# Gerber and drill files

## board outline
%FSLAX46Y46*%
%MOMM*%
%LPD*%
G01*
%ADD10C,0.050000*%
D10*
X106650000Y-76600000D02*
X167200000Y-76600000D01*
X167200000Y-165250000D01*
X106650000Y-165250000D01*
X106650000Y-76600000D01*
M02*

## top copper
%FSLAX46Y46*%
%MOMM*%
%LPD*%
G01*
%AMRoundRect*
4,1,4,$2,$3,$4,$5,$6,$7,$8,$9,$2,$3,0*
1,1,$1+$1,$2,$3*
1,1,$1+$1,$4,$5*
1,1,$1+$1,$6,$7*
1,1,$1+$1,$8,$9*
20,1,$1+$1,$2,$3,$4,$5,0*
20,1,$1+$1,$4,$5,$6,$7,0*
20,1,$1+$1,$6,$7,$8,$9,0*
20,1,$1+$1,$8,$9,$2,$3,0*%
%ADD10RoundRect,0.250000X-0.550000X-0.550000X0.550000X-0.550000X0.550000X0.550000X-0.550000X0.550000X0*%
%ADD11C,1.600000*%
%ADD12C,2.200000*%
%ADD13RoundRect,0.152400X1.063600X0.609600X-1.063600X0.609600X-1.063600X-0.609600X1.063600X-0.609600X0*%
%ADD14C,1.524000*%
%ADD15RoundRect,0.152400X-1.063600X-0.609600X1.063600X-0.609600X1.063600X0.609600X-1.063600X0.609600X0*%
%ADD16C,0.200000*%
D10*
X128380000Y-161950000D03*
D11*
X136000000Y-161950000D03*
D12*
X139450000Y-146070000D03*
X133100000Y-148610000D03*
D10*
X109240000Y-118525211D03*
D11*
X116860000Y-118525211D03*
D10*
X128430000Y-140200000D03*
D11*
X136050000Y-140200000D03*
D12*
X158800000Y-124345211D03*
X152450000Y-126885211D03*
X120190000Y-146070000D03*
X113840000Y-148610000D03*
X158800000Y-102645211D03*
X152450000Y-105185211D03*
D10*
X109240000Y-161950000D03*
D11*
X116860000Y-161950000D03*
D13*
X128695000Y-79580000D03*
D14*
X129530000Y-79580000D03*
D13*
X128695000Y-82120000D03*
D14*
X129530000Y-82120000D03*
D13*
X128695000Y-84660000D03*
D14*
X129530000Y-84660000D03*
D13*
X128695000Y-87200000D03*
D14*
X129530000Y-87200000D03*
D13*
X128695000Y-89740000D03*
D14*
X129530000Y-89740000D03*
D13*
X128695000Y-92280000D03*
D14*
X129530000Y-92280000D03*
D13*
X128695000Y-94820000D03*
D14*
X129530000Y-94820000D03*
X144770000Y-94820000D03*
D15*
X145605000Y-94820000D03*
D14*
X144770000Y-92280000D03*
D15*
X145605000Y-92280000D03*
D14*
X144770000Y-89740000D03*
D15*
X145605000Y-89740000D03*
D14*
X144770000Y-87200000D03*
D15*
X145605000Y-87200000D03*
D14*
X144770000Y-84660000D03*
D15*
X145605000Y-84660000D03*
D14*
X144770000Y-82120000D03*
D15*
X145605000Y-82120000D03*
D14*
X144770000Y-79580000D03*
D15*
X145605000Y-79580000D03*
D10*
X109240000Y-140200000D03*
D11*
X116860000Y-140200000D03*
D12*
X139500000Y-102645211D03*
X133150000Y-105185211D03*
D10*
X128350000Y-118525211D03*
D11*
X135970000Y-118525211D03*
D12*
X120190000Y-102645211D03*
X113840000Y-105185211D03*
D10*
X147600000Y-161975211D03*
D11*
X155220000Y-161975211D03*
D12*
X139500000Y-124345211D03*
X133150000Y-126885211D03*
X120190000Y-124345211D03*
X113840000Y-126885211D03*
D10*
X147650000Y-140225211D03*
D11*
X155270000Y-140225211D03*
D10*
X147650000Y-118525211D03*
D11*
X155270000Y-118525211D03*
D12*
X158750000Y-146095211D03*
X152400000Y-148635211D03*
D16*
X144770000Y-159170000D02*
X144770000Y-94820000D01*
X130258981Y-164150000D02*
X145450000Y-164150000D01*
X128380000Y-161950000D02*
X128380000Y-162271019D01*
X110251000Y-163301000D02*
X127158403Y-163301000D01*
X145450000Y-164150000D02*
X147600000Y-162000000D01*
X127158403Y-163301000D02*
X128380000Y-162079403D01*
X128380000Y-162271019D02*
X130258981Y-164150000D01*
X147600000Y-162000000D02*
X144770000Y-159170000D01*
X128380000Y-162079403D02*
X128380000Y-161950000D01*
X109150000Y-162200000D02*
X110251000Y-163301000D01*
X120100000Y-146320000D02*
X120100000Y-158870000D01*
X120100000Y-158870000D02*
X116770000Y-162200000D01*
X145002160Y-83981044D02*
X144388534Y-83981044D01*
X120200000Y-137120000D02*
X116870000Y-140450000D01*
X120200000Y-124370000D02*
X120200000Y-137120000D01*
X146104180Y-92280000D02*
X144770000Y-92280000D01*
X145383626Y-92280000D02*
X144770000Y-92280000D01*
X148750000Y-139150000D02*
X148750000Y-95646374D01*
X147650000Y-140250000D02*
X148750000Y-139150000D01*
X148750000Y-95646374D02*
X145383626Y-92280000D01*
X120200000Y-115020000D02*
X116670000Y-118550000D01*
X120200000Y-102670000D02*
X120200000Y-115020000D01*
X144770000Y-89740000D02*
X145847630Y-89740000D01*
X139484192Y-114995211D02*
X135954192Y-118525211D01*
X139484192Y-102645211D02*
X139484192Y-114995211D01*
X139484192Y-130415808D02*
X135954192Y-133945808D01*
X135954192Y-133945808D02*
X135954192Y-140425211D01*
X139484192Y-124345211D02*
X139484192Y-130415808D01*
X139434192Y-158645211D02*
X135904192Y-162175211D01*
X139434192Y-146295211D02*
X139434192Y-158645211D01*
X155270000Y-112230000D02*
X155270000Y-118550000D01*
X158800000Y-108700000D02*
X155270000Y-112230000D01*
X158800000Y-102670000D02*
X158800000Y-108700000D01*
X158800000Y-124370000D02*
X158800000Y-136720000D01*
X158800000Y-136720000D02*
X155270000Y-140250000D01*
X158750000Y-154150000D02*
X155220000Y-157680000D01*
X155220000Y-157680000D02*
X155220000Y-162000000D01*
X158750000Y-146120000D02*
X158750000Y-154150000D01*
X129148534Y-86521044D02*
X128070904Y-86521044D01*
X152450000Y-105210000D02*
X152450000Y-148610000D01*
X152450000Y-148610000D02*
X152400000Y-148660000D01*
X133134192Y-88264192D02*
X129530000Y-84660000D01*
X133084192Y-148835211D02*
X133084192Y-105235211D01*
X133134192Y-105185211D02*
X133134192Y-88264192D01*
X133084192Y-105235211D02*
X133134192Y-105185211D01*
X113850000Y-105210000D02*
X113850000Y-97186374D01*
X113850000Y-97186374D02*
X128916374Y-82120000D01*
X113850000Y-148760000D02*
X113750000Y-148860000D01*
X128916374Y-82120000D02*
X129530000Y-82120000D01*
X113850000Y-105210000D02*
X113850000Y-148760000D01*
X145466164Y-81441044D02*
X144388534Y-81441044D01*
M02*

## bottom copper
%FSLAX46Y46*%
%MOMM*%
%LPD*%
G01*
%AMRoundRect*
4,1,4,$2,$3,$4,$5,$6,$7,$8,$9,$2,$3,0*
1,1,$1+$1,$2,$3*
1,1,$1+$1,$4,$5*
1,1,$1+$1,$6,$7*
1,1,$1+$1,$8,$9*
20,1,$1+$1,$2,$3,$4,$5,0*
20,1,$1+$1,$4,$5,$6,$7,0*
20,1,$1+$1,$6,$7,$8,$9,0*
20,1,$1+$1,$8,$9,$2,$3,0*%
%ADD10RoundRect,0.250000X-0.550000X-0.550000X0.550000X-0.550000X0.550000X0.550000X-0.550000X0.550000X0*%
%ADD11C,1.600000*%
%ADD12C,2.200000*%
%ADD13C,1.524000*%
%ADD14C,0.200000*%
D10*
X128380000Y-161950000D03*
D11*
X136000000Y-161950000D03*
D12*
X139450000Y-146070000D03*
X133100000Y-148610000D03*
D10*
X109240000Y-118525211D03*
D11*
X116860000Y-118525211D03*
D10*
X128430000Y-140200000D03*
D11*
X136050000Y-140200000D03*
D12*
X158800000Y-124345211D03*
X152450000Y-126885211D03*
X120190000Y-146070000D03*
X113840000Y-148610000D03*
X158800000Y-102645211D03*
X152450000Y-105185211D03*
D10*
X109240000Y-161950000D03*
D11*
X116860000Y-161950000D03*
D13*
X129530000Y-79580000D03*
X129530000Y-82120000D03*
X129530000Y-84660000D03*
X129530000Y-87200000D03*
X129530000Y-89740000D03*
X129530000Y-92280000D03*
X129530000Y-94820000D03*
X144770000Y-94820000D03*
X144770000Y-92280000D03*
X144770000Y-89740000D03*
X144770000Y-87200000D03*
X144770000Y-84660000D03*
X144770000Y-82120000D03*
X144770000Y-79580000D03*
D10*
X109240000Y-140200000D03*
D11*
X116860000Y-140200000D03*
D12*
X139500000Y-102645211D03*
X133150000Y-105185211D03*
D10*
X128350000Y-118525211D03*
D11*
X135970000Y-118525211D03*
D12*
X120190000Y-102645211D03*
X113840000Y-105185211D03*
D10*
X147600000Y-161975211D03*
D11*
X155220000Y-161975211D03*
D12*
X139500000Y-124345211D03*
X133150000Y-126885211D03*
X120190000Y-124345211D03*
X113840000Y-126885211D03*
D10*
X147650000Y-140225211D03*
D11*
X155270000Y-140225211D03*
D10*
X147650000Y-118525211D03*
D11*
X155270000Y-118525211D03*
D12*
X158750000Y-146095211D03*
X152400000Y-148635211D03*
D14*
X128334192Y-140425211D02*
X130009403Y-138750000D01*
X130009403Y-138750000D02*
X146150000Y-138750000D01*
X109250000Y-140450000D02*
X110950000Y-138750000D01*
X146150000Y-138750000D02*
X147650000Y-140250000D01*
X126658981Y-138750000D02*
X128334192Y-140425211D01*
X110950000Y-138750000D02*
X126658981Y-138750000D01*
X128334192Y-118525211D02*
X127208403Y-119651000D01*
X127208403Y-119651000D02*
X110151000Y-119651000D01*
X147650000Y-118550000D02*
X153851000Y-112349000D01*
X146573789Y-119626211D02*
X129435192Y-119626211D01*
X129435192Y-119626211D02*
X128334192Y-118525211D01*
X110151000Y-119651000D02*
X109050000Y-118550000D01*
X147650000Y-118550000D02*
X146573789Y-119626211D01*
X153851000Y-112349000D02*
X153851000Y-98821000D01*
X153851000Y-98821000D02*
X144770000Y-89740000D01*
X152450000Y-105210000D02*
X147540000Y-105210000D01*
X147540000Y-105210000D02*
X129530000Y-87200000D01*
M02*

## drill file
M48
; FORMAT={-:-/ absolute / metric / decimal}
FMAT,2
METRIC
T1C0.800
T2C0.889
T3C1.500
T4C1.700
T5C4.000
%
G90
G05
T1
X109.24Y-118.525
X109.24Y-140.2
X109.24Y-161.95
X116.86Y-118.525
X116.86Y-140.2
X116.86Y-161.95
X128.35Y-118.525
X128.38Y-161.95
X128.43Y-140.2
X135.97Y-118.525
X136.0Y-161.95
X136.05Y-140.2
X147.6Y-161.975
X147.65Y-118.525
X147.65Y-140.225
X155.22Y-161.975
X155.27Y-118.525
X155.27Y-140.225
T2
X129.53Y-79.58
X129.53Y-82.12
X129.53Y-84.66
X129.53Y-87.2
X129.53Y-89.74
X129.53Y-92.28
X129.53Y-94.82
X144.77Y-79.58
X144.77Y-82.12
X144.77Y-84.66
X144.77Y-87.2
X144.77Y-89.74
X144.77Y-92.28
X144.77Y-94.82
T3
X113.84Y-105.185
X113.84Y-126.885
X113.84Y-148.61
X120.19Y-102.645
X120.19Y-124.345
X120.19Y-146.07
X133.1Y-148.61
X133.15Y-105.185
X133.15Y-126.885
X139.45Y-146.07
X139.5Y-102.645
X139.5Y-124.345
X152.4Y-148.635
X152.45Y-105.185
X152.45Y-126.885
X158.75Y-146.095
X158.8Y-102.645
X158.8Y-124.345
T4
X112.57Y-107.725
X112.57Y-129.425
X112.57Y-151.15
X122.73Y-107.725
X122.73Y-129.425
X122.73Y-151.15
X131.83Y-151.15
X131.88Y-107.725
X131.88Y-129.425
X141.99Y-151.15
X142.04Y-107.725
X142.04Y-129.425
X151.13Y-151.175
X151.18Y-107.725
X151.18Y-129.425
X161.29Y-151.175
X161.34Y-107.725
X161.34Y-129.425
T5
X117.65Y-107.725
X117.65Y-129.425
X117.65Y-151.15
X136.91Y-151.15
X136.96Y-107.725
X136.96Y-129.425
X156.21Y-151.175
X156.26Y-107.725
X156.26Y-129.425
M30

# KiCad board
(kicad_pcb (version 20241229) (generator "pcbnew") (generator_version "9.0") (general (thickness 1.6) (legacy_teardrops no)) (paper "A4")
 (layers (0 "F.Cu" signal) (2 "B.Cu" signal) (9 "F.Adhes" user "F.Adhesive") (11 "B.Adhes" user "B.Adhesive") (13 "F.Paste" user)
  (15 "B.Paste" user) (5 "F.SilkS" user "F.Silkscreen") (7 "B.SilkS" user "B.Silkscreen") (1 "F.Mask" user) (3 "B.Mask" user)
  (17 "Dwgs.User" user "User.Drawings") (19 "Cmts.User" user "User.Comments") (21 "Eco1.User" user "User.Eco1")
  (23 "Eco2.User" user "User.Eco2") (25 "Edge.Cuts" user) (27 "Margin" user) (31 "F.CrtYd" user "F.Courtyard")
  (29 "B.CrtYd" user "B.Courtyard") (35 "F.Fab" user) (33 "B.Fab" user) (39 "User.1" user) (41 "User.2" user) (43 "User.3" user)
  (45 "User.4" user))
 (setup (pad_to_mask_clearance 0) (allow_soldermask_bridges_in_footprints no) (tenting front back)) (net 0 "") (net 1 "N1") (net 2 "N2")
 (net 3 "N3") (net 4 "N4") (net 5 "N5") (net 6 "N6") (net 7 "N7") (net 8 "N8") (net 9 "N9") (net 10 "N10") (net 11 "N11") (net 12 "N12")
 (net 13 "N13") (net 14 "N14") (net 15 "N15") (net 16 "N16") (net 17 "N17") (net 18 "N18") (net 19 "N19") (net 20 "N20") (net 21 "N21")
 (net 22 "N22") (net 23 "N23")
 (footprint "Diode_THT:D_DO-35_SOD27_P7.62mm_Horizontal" (layer "F.Cu") (at 128.38 161.95)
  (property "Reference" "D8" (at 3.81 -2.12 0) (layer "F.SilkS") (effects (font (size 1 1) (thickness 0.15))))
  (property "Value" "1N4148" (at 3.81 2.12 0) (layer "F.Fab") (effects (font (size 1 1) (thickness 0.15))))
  (pad "1" thru_hole roundrect (at 0 0) (size 1.6 1.6) (drill 0.8) (layers "*.Cu" "*.Mask") (remove_unused_layers no)
   (roundrect_rratio 0.15625) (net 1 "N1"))
  (pad "2" thru_hole circle (at 7.62 0) (size 1.6 1.6) (drill 0.8) (layers "*.Cu" "*.Mask") (remove_unused_layers no) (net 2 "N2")))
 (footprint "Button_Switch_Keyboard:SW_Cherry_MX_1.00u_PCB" (layer "F.Cu") (at 139.45 146.07)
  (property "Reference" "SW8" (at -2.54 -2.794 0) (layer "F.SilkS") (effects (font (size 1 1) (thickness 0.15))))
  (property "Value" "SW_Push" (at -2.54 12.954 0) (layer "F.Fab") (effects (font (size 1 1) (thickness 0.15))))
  (pad "" np_thru_hole circle (at -7.62 5.08) (size 1.7 1.7) (drill 1.7) (layers "*.Cu" "*.Mask"))
  (pad "" np_thru_hole circle (at -2.54 5.08) (size 4 4) (drill 4) (layers "*.Cu" "*.Mask"))
  (pad "" np_thru_hole circle (at 2.54 5.08) (size 1.7 1.7) (drill 1.7) (layers "*.Cu" "*.Mask"))
  (pad "1" thru_hole circle (at 0 0) (size 2.2 2.2) (drill 1.5) (layers "*.Cu" "*.Mask") (remove_unused_layers no) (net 2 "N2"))
  (pad "2" thru_hole circle (at -6.35 2.54) (size 2.2 2.2) (drill 1.5) (layers "*.Cu" "*.Mask") (remove_unused_layers no) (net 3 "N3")))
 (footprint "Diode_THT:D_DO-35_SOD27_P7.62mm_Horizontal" (layer "F.Cu") (at 109.24 118.525211)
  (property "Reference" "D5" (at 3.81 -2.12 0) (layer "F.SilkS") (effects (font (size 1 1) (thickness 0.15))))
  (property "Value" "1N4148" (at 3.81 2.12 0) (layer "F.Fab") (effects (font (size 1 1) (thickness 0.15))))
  (pad "1" thru_hole roundrect (at 0 0) (size 1.6 1.6) (drill 0.8) (layers "*.Cu" "*.Mask") (remove_unused_layers no)
   (roundrect_rratio 0.15625) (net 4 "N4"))
  (pad "2" thru_hole circle (at 7.62 0) (size 1.6 1.6) (drill 0.8) (layers "*.Cu" "*.Mask") (remove_unused_layers no) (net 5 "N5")))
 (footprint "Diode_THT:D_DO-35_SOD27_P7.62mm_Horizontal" (layer "F.Cu") (at 128.43 140.2)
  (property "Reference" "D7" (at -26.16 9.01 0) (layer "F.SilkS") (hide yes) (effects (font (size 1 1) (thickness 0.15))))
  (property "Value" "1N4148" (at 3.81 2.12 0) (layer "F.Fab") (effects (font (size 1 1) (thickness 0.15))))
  (pad "1" thru_hole roundrect (at 0 0) (size 1.6 1.6) (drill 0.8) (layers "*.Cu" "*.Mask") (remove_unused_layers no)
   (roundrect_rratio 0.15625) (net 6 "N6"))
  (pad "2" thru_hole circle (at 7.62 0) (size 1.6 1.6) (drill 0.8) (layers "*.Cu" "*.Mask") (remove_unused_layers no) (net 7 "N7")))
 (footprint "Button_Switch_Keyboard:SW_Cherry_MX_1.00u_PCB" (layer "F.Cu") (at 158.8 124.345211)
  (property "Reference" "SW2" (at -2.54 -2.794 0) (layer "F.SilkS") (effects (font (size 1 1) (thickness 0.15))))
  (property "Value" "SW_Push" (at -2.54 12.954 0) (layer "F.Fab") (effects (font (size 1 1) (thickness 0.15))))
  (pad "" np_thru_hole circle (at -7.62 5.08) (size 1.7 1.7) (drill 1.7) (layers "*.Cu" "*.Mask"))
  (pad "" np_thru_hole circle (at -2.54 5.08) (size 4 4) (drill 4) (layers "*.Cu" "*.Mask"))
  (pad "" np_thru_hole circle (at 2.54 5.08) (size 1.7 1.7) (drill 1.7) (layers "*.Cu" "*.Mask"))
  (pad "1" thru_hole circle (at 0 0) (size 2.2 2.2) (drill 1.5) (layers "*.Cu" "*.Mask") (remove_unused_layers no) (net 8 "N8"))
  (pad "2" thru_hole circle (at -6.35 2.54) (size 2.2 2.2) (drill 1.5) (layers "*.Cu" "*.Mask") (remove_unused_layers no) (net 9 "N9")))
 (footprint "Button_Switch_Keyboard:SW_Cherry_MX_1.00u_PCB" (layer "F.Cu") (at 120.19 146.07)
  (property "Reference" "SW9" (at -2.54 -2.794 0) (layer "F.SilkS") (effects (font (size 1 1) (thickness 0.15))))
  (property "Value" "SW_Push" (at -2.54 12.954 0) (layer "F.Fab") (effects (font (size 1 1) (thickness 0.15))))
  (pad "" np_thru_hole circle (at -7.62 5.08) (size 1.7 1.7) (drill 1.7) (layers "*.Cu" "*.Mask"))
  (pad "" np_thru_hole circle (at -2.54 5.08) (size 4 4) (drill 4) (layers "*.Cu" "*.Mask"))
  (pad "" np_thru_hole circle (at 2.54 5.08) (size 1.7 1.7) (drill 1.7) (layers "*.Cu" "*.Mask"))
  (pad "1" thru_hole circle (at 0 0) (size 2.2 2.2) (drill 1.5) (layers "*.Cu" "*.Mask") (remove_unused_layers no) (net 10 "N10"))
  (pad "2" thru_hole circle (at -6.35 2.54) (size 2.2 2.2) (drill 1.5) (layers "*.Cu" "*.Mask") (remove_unused_layers no) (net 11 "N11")))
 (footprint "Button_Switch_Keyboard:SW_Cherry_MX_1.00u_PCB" (layer "F.Cu") (at 158.8 102.645211)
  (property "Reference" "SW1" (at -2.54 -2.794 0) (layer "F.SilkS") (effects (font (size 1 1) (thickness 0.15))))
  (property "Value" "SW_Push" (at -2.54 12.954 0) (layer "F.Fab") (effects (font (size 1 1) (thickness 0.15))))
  (pad "" np_thru_hole circle (at -7.62 5.08) (size 1.7 1.7) (drill 1.7) (layers "*.Cu" "*.Mask"))
  (pad "" np_thru_hole circle (at -2.54 5.08) (size 4 4) (drill 4) (layers "*.Cu" "*.Mask"))
  (pad "" np_thru_hole circle (at 2.54 5.08) (size 1.7 1.7) (drill 1.7) (layers "*.Cu" "*.Mask"))
  (pad "1" thru_hole circle (at 0 0) (size 2.2 2.2) (drill 1.5) (layers "*.Cu" "*.Mask") (remove_unused_layers no) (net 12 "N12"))
  (pad "2" thru_hole circle (at -6.35 2.54) (size 2.2 2.2) (drill 1.5) (layers "*.Cu" "*.Mask") (remove_unused_layers no) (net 9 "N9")))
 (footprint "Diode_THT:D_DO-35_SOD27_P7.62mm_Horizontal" (layer "F.Cu") (at 109.24 161.95)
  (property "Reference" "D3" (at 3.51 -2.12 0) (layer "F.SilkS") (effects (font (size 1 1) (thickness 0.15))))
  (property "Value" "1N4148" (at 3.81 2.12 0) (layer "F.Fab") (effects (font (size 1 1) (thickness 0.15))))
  (pad "1" thru_hole roundrect (at 0 0) (size 1.6 1.6) (drill 0.8) (layers "*.Cu" "*.Mask") (remove_unused_layers no)
   (roundrect_rratio 0.15625) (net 1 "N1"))
  (pad "2" thru_hole circle (at 7.62 0) (size 1.6 1.6) (drill 0.8) (layers "*.Cu" "*.Mask") (remove_unused_layers no) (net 10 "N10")))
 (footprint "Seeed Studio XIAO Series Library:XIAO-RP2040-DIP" (layer "F.Cu") (at 137.15 87.2)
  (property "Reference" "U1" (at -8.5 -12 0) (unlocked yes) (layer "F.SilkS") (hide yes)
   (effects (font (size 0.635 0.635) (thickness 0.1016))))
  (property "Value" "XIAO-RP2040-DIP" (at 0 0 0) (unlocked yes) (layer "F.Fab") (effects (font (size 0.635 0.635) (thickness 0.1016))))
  (pad "1" smd roundrect (at -8.455 -7.62 180) (size 2.432 1.524) (layers "F.Cu" "F.Mask") (roundrect_rratio 0.1) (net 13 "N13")
   (thermal_bridge_angle 45))
  (pad "1" thru_hole circle (at -7.62 -7.62 180) (size 1.524 1.524) (drill 0.889) (layers "*.Cu" "*.Mask") (remove_unused_layers no)
   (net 13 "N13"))
  (pad "2" smd roundrect (at -8.455 -5.08 180) (size 2.432 1.524) (layers "F.Cu" "F.Mask") (roundrect_rratio 0.1) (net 11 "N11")
   (thermal_bridge_angle 45))
  (pad "2" thru_hole circle (at -7.62 -5.08 180) (size 1.524 1.524) (drill 0.889) (layers "*.Cu" "*.Mask") (remove_unused_layers no)
   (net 11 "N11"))
  (pad "3" smd roundrect (at -8.455 -2.54 180) (size 2.432 1.524) (layers "F.Cu" "F.Mask") (roundrect_rratio 0.1) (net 3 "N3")
   (thermal_bridge_angle 45))
  (pad "3" thru_hole circle (at -7.62 -2.54 180) (size 1.524 1.524) (drill 0.889) (layers "*.Cu" "*.Mask") (remove_unused_layers no)
   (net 3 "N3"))
  (pad "4" smd roundrect (at -8.455 0 180) (size 2.432 1.524) (layers "F.Cu" "F.Mask") (roundrect_rratio 0.1) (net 9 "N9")
   (thermal_bridge_angle 45))
  (pad "4" thru_hole circle (at -7.62 0 180) (size 1.524 1.524) (drill 0.889) (layers "*.Cu" "*.Mask") (remove_unused_layers no)
   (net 9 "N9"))
  (pad "5" smd roundrect (at -8.455 2.54 180) (size 2.432 1.524) (layers "F.Cu" "F.Mask") (roundrect_rratio 0.1) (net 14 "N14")
   (thermal_bridge_angle 45))
  (pad "5" thru_hole circle (at -7.62 2.54 180) (size 1.524 1.524) (drill 0.889) (layers "*.Cu" "*.Mask") (remove_unused_layers no)
   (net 14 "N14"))
  (pad "6" smd roundrect (at -8.455 5.08 180) (size 2.432 1.524) (layers "F.Cu" "F.Mask") (roundrect_rratio 0.1) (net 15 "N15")
   (thermal_bridge_angle 45))
  (pad "6" thru_hole circle (at -7.62 5.08 180) (size 1.524 1.524) (drill 0.889) (layers "*.Cu" "*.Mask") (remove_unused_layers no)
   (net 15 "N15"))
  (pad "7" smd roundrect (at -8.455 7.62 180) (size 2.432 1.524) (layers "F.Cu" "F.Mask") (roundrect_rratio 0.1) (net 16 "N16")
   (thermal_bridge_angle 45))
  (pad "7" thru_hole circle (at -7.62 7.62 180) (size 1.524 1.524) (drill 0.889) (layers "*.Cu" "*.Mask") (remove_unused_layers no)
   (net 16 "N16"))
  (pad "8" thru_hole circle (at 7.62 7.62) (size 1.524 1.524) (drill 0.889) (layers "*.Cu" "*.Mask") (remove_unused_layers no) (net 1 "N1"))
  (pad "8" smd roundrect (at 8.455 7.62) (size 2.432 1.524) (layers "F.Cu" "F.Mask") (roundrect_rratio 0.1) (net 1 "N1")
   (thermal_bridge_angle 45))
  (pad "9" thru_hole circle (at 7.62 5.08) (size 1.524 1.524) (drill 0.889) (layers "*.Cu" "*.Mask") (remove_unused_layers no) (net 6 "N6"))
  (pad "9" smd roundrect (at 8.455 5.08) (size 2.432 1.524) (layers "F.Cu" "F.Mask") (roundrect_rratio 0.1) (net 6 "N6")
   (thermal_bridge_angle 45))
  (pad "10" thru_hole circle (at 7.62 2.54) (size 1.524 1.524) (drill 0.889) (layers "*.Cu" "*.Mask") (remove_unused_layers no) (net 4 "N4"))
  (pad "10" smd roundrect (at 8.455 2.54) (size 2.432 1.524) (layers "F.Cu" "F.Mask") (roundrect_rratio 0.1) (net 4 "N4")
   (thermal_bridge_angle 45))
  (pad "11" thru_hole circle (at 7.62 0) (size 1.524 1.524) (drill 0.889) (layers "*.Cu" "*.Mask") (remove_unused_layers no) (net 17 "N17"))
  (pad "11" smd roundrect (at 8.455 0) (size 2.432 1.524) (layers "F.Cu" "F.Mask") (roundrect_rratio 0.1) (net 17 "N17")
   (thermal_bridge_angle 45))
  (pad "12" thru_hole circle (at 7.62 -2.54) (size 1.524 1.524) (drill 0.889) (layers "*.Cu" "*.Mask") (remove_unused_layers no)
   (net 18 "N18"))
  (pad "12" smd roundrect (at 8.455 -2.54) (size 2.432 1.524) (layers "F.Cu" "F.Mask") (roundrect_rratio 0.1) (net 18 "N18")
   (thermal_bridge_angle 45))
  (pad "13" thru_hole circle (at 7.62 -5.08) (size 1.524 1.524) (drill 0.889) (layers "*.Cu" "*.Mask") (remove_unused_layers no)
   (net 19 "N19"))
  (pad "13" smd roundrect (at 8.455 -5.08) (size 2.432 1.524) (layers "F.Cu" "F.Mask") (roundrect_rratio 0.1) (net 19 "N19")
   (thermal_bridge_angle 45))
  (pad "14" thru_hole circle (at 7.62 -7.62) (size 1.524 1.524) (drill 0.889) (layers "*.Cu" "*.Mask") (remove_unused_layers no)
   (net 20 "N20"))
  (pad "14" smd roundrect (at 8.455 -7.62) (size 2.432 1.524) (layers "F.Cu" "F.Mask") (roundrect_rratio 0.1) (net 20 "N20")
   (thermal_bridge_angle 45)))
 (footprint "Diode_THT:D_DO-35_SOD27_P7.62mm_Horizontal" (layer "F.Cu") (at 109.24 140.2)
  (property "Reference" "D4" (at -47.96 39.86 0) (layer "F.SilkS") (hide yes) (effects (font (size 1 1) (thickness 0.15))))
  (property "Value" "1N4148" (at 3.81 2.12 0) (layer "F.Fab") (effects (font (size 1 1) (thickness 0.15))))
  (pad "1" thru_hole roundrect (at 0 0) (size 1.6 1.6) (drill 0.8) (layers "*.Cu" "*.Mask") (remove_unused_layers no)
   (roundrect_rratio 0.15625) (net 6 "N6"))
  (pad "2" thru_hole circle (at 7.62 0) (size 1.6 1.6) (drill 0.8) (layers "*.Cu" "*.Mask") (remove_unused_layers no) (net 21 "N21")))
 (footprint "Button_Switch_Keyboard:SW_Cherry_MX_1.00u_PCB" (layer "F.Cu") (at 139.5 102.645211)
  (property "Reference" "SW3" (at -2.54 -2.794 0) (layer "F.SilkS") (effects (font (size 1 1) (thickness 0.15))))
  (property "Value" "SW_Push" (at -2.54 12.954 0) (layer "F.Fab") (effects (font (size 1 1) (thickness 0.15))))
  (pad "" np_thru_hole circle (at -7.62 5.08) (size 1.7 1.7) (drill 1.7) (layers "*.Cu" "*.Mask"))
  (pad "" np_thru_hole circle (at -2.54 5.08) (size 4 4) (drill 4) (layers "*.Cu" "*.Mask"))
  (pad "" np_thru_hole circle (at 2.54 5.08) (size 1.7 1.7) (drill 1.7) (layers "*.Cu" "*.Mask"))
  (pad "1" thru_hole circle (at 0 0) (size 2.2 2.2) (drill 1.5) (layers "*.Cu" "*.Mask") (remove_unused_layers no) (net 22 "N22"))
  (pad "2" thru_hole circle (at -6.35 2.54) (size 2.2 2.2) (drill 1.5) (layers "*.Cu" "*.Mask") (remove_unused_layers no) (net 3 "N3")))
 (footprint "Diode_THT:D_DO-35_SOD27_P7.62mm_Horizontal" (layer "F.Cu") (at 128.35 118.525211)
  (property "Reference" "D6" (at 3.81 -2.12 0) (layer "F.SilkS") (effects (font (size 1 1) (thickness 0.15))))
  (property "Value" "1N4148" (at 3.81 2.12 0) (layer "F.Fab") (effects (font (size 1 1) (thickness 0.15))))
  (pad "1" thru_hole roundrect (at 0 0) (size 1.6 1.6) (drill 0.8) (layers "*.Cu" "*.Mask") (remove_unused_layers no)
   (roundrect_rratio 0.15625) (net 4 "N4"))
  (pad "2" thru_hole circle (at 7.62 0) (size 1.6 1.6) (drill 0.8) (layers "*.Cu" "*.Mask") (remove_unused_layers no) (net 22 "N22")))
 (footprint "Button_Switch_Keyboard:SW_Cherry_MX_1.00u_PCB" (layer "F.Cu") (at 120.19 102.645211)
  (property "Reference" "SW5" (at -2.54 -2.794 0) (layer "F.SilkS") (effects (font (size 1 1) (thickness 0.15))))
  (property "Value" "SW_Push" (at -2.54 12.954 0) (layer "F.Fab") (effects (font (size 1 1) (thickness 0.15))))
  (pad "" np_thru_hole circle (at -7.62 5.08) (size 1.7 1.7) (drill 1.7) (layers "*.Cu" "*.Mask"))
  (pad "" np_thru_hole circle (at -2.54 5.08) (size 4 4) (drill 4) (layers "*.Cu" "*.Mask"))
  (pad "" np_thru_hole circle (at 2.54 5.08) (size 1.7 1.7) (drill 1.7) (layers "*.Cu" "*.Mask"))
  (pad "1" thru_hole circle (at 0 0) (size 2.2 2.2) (drill 1.5) (layers "*.Cu" "*.Mask") (remove_unused_layers no) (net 5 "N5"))
  (pad "2" thru_hole circle (at -6.35 2.54) (size 2.2 2.2) (drill 1.5) (layers "*.Cu" "*.Mask") (remove_unused_layers no) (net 11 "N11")))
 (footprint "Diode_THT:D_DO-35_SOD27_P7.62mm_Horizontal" (layer "F.Cu") (at 147.6 161.975211)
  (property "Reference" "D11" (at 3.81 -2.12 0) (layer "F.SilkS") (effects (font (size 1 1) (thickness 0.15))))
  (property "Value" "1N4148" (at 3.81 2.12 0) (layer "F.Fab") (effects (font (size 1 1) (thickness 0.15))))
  (pad "1" thru_hole roundrect (at 0 0) (size 1.6 1.6) (drill 0.8) (layers "*.Cu" "*.Mask") (remove_unused_layers no)
   (roundrect_rratio 0.15625) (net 1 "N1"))
  (pad "2" thru_hole circle (at 7.62 0) (size 1.6 1.6) (drill 0.8) (layers "*.Cu" "*.Mask") (remove_unused_layers no) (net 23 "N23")))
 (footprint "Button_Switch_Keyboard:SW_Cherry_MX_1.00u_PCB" (layer "F.Cu") (at 139.5 124.345211)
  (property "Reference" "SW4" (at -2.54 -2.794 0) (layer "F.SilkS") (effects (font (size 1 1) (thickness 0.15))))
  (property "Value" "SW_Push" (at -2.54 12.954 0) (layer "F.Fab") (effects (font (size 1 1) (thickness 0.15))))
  (pad "" np_thru_hole circle (at -7.62 5.08) (size 1.7 1.7) (drill 1.7) (layers "*.Cu" "*.Mask"))
  (pad "" np_thru_hole circle (at -2.54 5.08) (size 4 4) (drill 4) (layers "*.Cu" "*.Mask"))
  (pad "" np_thru_hole circle (at 2.54 5.08) (size 1.7 1.7) (drill 1.7) (layers "*.Cu" "*.Mask"))
  (pad "1" thru_hole circle (at 0 0) (size 2.2 2.2) (drill 1.5) (layers "*.Cu" "*.Mask") (remove_unused_layers no) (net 7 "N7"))
  (pad "2" thru_hole circle (at -6.35 2.54) (size 2.2 2.2) (drill 1.5) (layers "*.Cu" "*.Mask") (remove_unused_layers no) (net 3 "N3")))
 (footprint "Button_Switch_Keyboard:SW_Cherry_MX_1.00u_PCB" (layer "F.Cu") (at 120.19 124.345211)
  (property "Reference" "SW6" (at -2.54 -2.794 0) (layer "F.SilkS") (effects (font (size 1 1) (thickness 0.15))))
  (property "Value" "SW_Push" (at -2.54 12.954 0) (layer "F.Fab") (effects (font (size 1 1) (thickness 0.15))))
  (pad "" np_thru_hole circle (at -7.62 5.08) (size 1.7 1.7) (drill 1.7) (layers "*.Cu" "*.Mask"))
  (pad "" np_thru_hole circle (at -2.54 5.08) (size 4 4) (drill 4) (layers "*.Cu" "*.Mask"))
  (pad "" np_thru_hole circle (at 2.54 5.08) (size 1.7 1.7) (drill 1.7) (layers "*.Cu" "*.Mask"))
  (pad "1" thru_hole circle (at 0 0) (size 2.2 2.2) (drill 1.5) (layers "*.Cu" "*.Mask") (remove_unused_layers no) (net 21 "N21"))
  (pad "2" thru_hole circle (at -6.35 2.54) (size 2.2 2.2) (drill 1.5) (layers "*.Cu" "*.Mask") (remove_unused_layers no) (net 11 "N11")))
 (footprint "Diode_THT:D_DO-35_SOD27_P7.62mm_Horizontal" (layer "F.Cu") (at 147.65 140.225211)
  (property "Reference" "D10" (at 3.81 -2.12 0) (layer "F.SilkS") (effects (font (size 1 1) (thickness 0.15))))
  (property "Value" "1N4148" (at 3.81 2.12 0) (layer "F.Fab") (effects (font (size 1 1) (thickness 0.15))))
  (pad "1" thru_hole roundrect (at 0 0) (size 1.6 1.6) (drill 0.8) (layers "*.Cu" "*.Mask") (remove_unused_layers no)
   (roundrect_rratio 0.15625) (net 6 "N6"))
  (pad "2" thru_hole circle (at 7.62 0) (size 1.6 1.6) (drill 0.8) (layers "*.Cu" "*.Mask") (remove_unused_layers no) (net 8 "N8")))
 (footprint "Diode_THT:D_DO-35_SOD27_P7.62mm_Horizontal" (layer "F.Cu") (at 147.65 118.525211)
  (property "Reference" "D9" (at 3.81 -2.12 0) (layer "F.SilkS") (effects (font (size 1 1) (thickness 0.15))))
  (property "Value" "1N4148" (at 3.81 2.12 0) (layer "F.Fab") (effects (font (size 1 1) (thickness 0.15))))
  (pad "1" thru_hole roundrect (at 0 0) (size 1.6 1.6) (drill 0.8) (layers "*.Cu" "*.Mask") (remove_unused_layers no)
   (roundrect_rratio 0.15625) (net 4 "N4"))
  (pad "2" thru_hole circle (at 7.62 0) (size 1.6 1.6) (drill 0.8) (layers "*.Cu" "*.Mask") (remove_unused_layers no) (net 12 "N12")))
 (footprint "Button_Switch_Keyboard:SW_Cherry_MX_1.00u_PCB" (layer "F.Cu") (at 158.75 146.095211)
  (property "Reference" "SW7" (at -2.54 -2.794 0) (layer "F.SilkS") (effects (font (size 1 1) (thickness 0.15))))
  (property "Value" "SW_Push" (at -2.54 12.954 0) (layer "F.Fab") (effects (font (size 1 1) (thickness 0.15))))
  (pad "" np_thru_hole circle (at -7.62 5.08) (size 1.7 1.7) (drill 1.7) (layers "*.Cu" "*.Mask"))
  (pad "" np_thru_hole circle (at -2.54 5.08) (size 4 4) (drill 4) (layers "*.Cu" "*.Mask"))
  (pad "" np_thru_hole circle (at 2.54 5.08) (size 1.7 1.7) (drill 1.7) (layers "*.Cu" "*.Mask"))
  (pad "1" thru_hole circle (at 0 0) (size 2.2 2.2) (drill 1.5) (layers "*.Cu" "*.Mask") (remove_unused_layers no) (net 23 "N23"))
  (pad "2" thru_hole circle (at -6.35 2.54) (size 2.2 2.2) (drill 1.5) (layers "*.Cu" "*.Mask") (remove_unused_layers no) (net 9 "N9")))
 (gr_rect (start 106.65 76.6) (end 167.2 165.25) (stroke (width 0.05) (type default)) (fill no) (layer "Edge.Cuts"))
 (segment (start 144.77 159.17) (end 144.77 94.82) (width 0.2) (layer "F.Cu") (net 1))
 (segment (start 130.258981 164.15) (end 145.45 164.15) (width 0.2) (layer "F.Cu") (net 1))
 (segment (start 128.38 161.95) (end 128.38 162.271019) (width 0.2) (layer "F.Cu") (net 1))
 (segment (start 110.251 163.301) (end 127.158403 163.301) (width 0.2) (layer "F.Cu") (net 1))
 (segment (start 145.45 164.15) (end 147.6 162) (width 0.2) (layer "F.Cu") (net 1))
 (segment (start 127.158403 163.301) (end 128.38 162.079403) (width 0.2) (layer "F.Cu") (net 1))
 (segment (start 128.38 162.271019) (end 130.258981 164.15) (width 0.2) (layer "F.Cu") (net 1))
 (segment (start 147.6 162) (end 144.77 159.17) (width 0.2) (layer "F.Cu") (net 1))
 (segment (start 128.38 162.079403) (end 128.38 161.95) (width 0.2) (layer "F.Cu") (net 1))
 (segment (start 109.15 162.2) (end 110.251 163.301) (width 0.2) (layer "F.Cu") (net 1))
 (segment (start 120.1 146.32) (end 120.1 158.87) (width 0.2) (layer "F.Cu") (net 10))
 (segment (start 120.1 158.87) (end 116.77 162.2) (width 0.2) (layer "F.Cu") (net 10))
 (segment (start 145.00216 83.981044) (end 144.388534 83.981044) (width 0.2) (layer "F.Cu") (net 18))
 (segment (start 120.2 137.12) (end 116.87 140.45) (width 0.2) (layer "F.Cu") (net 21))
 (segment (start 120.2 124.37) (end 120.2 137.12) (width 0.2) (layer "F.Cu") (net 21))
 (segment (start 146.10418 92.28) (end 144.77 92.28) (width 0.2) (layer "F.Cu") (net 6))
 (segment (start 145.383626 92.28) (end 144.77 92.28) (width 0.2) (layer "F.Cu") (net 6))
 (segment (start 148.75 139.15) (end 148.75 95.646374) (width 0.2) (layer "F.Cu") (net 6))
 (segment (start 147.65 140.25) (end 148.75 139.15) (width 0.2) (layer "F.Cu") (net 6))
 (segment (start 148.75 95.646374) (end 145.383626 92.28) (width 0.2) (layer "F.Cu") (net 6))
 (segment (start 128.334192 140.425211) (end 130.009403 138.75) (width 0.2) (layer "B.Cu") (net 6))
 (segment (start 130.009403 138.75) (end 146.15 138.75) (width 0.2) (layer "B.Cu") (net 6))
 (segment (start 109.25 140.45) (end 110.95 138.75) (width 0.2) (layer "B.Cu") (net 6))
 (segment (start 146.15 138.75) (end 147.65 140.25) (width 0.2) (layer "B.Cu") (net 6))
 (segment (start 126.658981 138.75) (end 128.334192 140.425211) (width 0.2) (layer "B.Cu") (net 6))
 (segment (start 110.95 138.75) (end 126.658981 138.75) (width 0.2) (layer "B.Cu") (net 6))
 (segment (start 120.2 115.02) (end 116.67 118.55) (width 0.2) (layer "F.Cu") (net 5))
 (segment (start 120.2 102.67) (end 120.2 115.02) (width 0.2) (layer "F.Cu") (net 5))
 (segment (start 144.77 89.74) (end 145.84763 89.74) (width 0.2) (layer "F.Cu") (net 4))
 (segment (start 128.334192 118.525211) (end 127.208403 119.651) (width 0.2) (layer "B.Cu") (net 4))
 (segment (start 127.208403 119.651) (end 110.151 119.651) (width 0.2) (layer "B.Cu") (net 4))
 (segment (start 147.65 118.55) (end 153.851 112.349) (width 0.2) (layer "B.Cu") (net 4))
 (segment (start 146.573789 119.626211) (end 129.435192 119.626211) (width 0.2) (layer "B.Cu") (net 4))
 (segment (start 129.435192 119.626211) (end 128.334192 118.525211) (width 0.2) (layer "B.Cu") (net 4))
 (segment (start 110.151 119.651) (end 109.05 118.55) (width 0.2) (layer "B.Cu") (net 4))
 (segment (start 147.65 118.55) (end 146.573789 119.626211) (width 0.2) (layer "B.Cu") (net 4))
 (segment (start 153.851 112.349) (end 153.851 98.821) (width 0.2) (layer "B.Cu") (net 4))
 (segment (start 153.851 98.821) (end 144.77 89.74) (width 0.2) (layer "B.Cu") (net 4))
 (segment (start 139.484192 114.995211) (end 135.954192 118.525211) (width 0.2) (layer "F.Cu") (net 22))
 (segment (start 139.484192 102.645211) (end 139.484192 114.995211) (width 0.2) (layer "F.Cu") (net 22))
 (segment (start 139.484192 130.415808) (end 135.954192 133.945808) (width 0.2) (layer "F.Cu") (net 7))
 (segment (start 135.954192 133.945808) (end 135.954192 140.425211) (width 0.2) (layer "F.Cu") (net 7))
 (segment (start 139.484192 124.345211) (end 139.484192 130.415808) (width 0.2) (layer "F.Cu") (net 7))
 (segment (start 139.434192 158.645211) (end 135.904192 162.175211) (width 0.2) (layer "F.Cu") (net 2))
 (segment (start 139.434192 146.295211) (end 139.434192 158.645211) (width 0.2) (layer "F.Cu") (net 2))
 (segment (start 155.27 112.23) (end 155.27 118.55) (width 0.2) (layer "F.Cu") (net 12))
 (segment (start 158.8 108.7) (end 155.27 112.23) (width 0.2) (layer "F.Cu") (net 12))
 (segment (start 158.8 102.67) (end 158.8 108.7) (width 0.2) (layer "F.Cu") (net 12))
 (segment (start 158.8 124.37) (end 158.8 136.72) (width 0.2) (layer "F.Cu") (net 8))
 (segment (start 158.8 136.72) (end 155.27 140.25) (width 0.2) (layer "F.Cu") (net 8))
 (segment (start 158.75 154.15) (end 155.22 157.68) (width 0.2) (layer "F.Cu") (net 23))
 (segment (start 155.22 157.68) (end 155.22 162) (width 0.2) (layer "F.Cu") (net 23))
 (segment (start 158.75 146.12) (end 158.75 154.15) (width 0.2) (layer "F.Cu") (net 23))
 (segment (start 129.148534 86.521044) (end 128.070904 86.521044) (width 0.2) (layer "F.Cu") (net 9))
 (segment (start 152.45 105.21) (end 152.45 148.61) (width 0.2) (layer "F.Cu") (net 9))
 (segment (start 152.45 148.61) (end 152.4 148.66) (width 0.2) (layer "F.Cu") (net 9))
 (segment (start 152.45 105.21) (end 147.54 105.21) (width 0.2) (layer "B.Cu") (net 9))
 (segment (start 147.54 105.21) (end 129.53 87.2) (width 0.2) (layer "B.Cu") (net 9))
 (segment (start 133.134192 88.264192) (end 129.53 84.66) (width 0.2) (layer "F.Cu") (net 3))
 (segment (start 133.084192 148.835211) (end 133.084192 105.235211) (width 0.2) (layer "F.Cu") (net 3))
 (segment (start 133.134192 105.185211) (end 133.134192 88.264192) (width 0.2) (layer "F.Cu") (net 3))
 (segment (start 133.084192 105.235211) (end 133.134192 105.185211) (width 0.2) (layer "F.Cu") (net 3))
 (segment (start 113.85 105.21) (end 113.85 97.186374) (width 0.2) (layer "F.Cu") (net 11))
 (segment (start 113.85 97.186374) (end 128.916374 82.12) (width 0.2) (layer "F.Cu") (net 11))
 (segment (start 113.85 148.76) (end 113.75 148.86) (width 0.2) (layer "F.Cu") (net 11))
 (segment (start 128.916374 82.12) (end 129.53 82.12) (width 0.2) (layer "F.Cu") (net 11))
 (segment (start 113.85 105.21) (end 113.85 148.76) (width 0.2) (layer "F.Cu") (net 11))
 (segment (start 145.466164 81.441044) (end 144.388534 81.441044) (width 0.2) (layer "F.Cu") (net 19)))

